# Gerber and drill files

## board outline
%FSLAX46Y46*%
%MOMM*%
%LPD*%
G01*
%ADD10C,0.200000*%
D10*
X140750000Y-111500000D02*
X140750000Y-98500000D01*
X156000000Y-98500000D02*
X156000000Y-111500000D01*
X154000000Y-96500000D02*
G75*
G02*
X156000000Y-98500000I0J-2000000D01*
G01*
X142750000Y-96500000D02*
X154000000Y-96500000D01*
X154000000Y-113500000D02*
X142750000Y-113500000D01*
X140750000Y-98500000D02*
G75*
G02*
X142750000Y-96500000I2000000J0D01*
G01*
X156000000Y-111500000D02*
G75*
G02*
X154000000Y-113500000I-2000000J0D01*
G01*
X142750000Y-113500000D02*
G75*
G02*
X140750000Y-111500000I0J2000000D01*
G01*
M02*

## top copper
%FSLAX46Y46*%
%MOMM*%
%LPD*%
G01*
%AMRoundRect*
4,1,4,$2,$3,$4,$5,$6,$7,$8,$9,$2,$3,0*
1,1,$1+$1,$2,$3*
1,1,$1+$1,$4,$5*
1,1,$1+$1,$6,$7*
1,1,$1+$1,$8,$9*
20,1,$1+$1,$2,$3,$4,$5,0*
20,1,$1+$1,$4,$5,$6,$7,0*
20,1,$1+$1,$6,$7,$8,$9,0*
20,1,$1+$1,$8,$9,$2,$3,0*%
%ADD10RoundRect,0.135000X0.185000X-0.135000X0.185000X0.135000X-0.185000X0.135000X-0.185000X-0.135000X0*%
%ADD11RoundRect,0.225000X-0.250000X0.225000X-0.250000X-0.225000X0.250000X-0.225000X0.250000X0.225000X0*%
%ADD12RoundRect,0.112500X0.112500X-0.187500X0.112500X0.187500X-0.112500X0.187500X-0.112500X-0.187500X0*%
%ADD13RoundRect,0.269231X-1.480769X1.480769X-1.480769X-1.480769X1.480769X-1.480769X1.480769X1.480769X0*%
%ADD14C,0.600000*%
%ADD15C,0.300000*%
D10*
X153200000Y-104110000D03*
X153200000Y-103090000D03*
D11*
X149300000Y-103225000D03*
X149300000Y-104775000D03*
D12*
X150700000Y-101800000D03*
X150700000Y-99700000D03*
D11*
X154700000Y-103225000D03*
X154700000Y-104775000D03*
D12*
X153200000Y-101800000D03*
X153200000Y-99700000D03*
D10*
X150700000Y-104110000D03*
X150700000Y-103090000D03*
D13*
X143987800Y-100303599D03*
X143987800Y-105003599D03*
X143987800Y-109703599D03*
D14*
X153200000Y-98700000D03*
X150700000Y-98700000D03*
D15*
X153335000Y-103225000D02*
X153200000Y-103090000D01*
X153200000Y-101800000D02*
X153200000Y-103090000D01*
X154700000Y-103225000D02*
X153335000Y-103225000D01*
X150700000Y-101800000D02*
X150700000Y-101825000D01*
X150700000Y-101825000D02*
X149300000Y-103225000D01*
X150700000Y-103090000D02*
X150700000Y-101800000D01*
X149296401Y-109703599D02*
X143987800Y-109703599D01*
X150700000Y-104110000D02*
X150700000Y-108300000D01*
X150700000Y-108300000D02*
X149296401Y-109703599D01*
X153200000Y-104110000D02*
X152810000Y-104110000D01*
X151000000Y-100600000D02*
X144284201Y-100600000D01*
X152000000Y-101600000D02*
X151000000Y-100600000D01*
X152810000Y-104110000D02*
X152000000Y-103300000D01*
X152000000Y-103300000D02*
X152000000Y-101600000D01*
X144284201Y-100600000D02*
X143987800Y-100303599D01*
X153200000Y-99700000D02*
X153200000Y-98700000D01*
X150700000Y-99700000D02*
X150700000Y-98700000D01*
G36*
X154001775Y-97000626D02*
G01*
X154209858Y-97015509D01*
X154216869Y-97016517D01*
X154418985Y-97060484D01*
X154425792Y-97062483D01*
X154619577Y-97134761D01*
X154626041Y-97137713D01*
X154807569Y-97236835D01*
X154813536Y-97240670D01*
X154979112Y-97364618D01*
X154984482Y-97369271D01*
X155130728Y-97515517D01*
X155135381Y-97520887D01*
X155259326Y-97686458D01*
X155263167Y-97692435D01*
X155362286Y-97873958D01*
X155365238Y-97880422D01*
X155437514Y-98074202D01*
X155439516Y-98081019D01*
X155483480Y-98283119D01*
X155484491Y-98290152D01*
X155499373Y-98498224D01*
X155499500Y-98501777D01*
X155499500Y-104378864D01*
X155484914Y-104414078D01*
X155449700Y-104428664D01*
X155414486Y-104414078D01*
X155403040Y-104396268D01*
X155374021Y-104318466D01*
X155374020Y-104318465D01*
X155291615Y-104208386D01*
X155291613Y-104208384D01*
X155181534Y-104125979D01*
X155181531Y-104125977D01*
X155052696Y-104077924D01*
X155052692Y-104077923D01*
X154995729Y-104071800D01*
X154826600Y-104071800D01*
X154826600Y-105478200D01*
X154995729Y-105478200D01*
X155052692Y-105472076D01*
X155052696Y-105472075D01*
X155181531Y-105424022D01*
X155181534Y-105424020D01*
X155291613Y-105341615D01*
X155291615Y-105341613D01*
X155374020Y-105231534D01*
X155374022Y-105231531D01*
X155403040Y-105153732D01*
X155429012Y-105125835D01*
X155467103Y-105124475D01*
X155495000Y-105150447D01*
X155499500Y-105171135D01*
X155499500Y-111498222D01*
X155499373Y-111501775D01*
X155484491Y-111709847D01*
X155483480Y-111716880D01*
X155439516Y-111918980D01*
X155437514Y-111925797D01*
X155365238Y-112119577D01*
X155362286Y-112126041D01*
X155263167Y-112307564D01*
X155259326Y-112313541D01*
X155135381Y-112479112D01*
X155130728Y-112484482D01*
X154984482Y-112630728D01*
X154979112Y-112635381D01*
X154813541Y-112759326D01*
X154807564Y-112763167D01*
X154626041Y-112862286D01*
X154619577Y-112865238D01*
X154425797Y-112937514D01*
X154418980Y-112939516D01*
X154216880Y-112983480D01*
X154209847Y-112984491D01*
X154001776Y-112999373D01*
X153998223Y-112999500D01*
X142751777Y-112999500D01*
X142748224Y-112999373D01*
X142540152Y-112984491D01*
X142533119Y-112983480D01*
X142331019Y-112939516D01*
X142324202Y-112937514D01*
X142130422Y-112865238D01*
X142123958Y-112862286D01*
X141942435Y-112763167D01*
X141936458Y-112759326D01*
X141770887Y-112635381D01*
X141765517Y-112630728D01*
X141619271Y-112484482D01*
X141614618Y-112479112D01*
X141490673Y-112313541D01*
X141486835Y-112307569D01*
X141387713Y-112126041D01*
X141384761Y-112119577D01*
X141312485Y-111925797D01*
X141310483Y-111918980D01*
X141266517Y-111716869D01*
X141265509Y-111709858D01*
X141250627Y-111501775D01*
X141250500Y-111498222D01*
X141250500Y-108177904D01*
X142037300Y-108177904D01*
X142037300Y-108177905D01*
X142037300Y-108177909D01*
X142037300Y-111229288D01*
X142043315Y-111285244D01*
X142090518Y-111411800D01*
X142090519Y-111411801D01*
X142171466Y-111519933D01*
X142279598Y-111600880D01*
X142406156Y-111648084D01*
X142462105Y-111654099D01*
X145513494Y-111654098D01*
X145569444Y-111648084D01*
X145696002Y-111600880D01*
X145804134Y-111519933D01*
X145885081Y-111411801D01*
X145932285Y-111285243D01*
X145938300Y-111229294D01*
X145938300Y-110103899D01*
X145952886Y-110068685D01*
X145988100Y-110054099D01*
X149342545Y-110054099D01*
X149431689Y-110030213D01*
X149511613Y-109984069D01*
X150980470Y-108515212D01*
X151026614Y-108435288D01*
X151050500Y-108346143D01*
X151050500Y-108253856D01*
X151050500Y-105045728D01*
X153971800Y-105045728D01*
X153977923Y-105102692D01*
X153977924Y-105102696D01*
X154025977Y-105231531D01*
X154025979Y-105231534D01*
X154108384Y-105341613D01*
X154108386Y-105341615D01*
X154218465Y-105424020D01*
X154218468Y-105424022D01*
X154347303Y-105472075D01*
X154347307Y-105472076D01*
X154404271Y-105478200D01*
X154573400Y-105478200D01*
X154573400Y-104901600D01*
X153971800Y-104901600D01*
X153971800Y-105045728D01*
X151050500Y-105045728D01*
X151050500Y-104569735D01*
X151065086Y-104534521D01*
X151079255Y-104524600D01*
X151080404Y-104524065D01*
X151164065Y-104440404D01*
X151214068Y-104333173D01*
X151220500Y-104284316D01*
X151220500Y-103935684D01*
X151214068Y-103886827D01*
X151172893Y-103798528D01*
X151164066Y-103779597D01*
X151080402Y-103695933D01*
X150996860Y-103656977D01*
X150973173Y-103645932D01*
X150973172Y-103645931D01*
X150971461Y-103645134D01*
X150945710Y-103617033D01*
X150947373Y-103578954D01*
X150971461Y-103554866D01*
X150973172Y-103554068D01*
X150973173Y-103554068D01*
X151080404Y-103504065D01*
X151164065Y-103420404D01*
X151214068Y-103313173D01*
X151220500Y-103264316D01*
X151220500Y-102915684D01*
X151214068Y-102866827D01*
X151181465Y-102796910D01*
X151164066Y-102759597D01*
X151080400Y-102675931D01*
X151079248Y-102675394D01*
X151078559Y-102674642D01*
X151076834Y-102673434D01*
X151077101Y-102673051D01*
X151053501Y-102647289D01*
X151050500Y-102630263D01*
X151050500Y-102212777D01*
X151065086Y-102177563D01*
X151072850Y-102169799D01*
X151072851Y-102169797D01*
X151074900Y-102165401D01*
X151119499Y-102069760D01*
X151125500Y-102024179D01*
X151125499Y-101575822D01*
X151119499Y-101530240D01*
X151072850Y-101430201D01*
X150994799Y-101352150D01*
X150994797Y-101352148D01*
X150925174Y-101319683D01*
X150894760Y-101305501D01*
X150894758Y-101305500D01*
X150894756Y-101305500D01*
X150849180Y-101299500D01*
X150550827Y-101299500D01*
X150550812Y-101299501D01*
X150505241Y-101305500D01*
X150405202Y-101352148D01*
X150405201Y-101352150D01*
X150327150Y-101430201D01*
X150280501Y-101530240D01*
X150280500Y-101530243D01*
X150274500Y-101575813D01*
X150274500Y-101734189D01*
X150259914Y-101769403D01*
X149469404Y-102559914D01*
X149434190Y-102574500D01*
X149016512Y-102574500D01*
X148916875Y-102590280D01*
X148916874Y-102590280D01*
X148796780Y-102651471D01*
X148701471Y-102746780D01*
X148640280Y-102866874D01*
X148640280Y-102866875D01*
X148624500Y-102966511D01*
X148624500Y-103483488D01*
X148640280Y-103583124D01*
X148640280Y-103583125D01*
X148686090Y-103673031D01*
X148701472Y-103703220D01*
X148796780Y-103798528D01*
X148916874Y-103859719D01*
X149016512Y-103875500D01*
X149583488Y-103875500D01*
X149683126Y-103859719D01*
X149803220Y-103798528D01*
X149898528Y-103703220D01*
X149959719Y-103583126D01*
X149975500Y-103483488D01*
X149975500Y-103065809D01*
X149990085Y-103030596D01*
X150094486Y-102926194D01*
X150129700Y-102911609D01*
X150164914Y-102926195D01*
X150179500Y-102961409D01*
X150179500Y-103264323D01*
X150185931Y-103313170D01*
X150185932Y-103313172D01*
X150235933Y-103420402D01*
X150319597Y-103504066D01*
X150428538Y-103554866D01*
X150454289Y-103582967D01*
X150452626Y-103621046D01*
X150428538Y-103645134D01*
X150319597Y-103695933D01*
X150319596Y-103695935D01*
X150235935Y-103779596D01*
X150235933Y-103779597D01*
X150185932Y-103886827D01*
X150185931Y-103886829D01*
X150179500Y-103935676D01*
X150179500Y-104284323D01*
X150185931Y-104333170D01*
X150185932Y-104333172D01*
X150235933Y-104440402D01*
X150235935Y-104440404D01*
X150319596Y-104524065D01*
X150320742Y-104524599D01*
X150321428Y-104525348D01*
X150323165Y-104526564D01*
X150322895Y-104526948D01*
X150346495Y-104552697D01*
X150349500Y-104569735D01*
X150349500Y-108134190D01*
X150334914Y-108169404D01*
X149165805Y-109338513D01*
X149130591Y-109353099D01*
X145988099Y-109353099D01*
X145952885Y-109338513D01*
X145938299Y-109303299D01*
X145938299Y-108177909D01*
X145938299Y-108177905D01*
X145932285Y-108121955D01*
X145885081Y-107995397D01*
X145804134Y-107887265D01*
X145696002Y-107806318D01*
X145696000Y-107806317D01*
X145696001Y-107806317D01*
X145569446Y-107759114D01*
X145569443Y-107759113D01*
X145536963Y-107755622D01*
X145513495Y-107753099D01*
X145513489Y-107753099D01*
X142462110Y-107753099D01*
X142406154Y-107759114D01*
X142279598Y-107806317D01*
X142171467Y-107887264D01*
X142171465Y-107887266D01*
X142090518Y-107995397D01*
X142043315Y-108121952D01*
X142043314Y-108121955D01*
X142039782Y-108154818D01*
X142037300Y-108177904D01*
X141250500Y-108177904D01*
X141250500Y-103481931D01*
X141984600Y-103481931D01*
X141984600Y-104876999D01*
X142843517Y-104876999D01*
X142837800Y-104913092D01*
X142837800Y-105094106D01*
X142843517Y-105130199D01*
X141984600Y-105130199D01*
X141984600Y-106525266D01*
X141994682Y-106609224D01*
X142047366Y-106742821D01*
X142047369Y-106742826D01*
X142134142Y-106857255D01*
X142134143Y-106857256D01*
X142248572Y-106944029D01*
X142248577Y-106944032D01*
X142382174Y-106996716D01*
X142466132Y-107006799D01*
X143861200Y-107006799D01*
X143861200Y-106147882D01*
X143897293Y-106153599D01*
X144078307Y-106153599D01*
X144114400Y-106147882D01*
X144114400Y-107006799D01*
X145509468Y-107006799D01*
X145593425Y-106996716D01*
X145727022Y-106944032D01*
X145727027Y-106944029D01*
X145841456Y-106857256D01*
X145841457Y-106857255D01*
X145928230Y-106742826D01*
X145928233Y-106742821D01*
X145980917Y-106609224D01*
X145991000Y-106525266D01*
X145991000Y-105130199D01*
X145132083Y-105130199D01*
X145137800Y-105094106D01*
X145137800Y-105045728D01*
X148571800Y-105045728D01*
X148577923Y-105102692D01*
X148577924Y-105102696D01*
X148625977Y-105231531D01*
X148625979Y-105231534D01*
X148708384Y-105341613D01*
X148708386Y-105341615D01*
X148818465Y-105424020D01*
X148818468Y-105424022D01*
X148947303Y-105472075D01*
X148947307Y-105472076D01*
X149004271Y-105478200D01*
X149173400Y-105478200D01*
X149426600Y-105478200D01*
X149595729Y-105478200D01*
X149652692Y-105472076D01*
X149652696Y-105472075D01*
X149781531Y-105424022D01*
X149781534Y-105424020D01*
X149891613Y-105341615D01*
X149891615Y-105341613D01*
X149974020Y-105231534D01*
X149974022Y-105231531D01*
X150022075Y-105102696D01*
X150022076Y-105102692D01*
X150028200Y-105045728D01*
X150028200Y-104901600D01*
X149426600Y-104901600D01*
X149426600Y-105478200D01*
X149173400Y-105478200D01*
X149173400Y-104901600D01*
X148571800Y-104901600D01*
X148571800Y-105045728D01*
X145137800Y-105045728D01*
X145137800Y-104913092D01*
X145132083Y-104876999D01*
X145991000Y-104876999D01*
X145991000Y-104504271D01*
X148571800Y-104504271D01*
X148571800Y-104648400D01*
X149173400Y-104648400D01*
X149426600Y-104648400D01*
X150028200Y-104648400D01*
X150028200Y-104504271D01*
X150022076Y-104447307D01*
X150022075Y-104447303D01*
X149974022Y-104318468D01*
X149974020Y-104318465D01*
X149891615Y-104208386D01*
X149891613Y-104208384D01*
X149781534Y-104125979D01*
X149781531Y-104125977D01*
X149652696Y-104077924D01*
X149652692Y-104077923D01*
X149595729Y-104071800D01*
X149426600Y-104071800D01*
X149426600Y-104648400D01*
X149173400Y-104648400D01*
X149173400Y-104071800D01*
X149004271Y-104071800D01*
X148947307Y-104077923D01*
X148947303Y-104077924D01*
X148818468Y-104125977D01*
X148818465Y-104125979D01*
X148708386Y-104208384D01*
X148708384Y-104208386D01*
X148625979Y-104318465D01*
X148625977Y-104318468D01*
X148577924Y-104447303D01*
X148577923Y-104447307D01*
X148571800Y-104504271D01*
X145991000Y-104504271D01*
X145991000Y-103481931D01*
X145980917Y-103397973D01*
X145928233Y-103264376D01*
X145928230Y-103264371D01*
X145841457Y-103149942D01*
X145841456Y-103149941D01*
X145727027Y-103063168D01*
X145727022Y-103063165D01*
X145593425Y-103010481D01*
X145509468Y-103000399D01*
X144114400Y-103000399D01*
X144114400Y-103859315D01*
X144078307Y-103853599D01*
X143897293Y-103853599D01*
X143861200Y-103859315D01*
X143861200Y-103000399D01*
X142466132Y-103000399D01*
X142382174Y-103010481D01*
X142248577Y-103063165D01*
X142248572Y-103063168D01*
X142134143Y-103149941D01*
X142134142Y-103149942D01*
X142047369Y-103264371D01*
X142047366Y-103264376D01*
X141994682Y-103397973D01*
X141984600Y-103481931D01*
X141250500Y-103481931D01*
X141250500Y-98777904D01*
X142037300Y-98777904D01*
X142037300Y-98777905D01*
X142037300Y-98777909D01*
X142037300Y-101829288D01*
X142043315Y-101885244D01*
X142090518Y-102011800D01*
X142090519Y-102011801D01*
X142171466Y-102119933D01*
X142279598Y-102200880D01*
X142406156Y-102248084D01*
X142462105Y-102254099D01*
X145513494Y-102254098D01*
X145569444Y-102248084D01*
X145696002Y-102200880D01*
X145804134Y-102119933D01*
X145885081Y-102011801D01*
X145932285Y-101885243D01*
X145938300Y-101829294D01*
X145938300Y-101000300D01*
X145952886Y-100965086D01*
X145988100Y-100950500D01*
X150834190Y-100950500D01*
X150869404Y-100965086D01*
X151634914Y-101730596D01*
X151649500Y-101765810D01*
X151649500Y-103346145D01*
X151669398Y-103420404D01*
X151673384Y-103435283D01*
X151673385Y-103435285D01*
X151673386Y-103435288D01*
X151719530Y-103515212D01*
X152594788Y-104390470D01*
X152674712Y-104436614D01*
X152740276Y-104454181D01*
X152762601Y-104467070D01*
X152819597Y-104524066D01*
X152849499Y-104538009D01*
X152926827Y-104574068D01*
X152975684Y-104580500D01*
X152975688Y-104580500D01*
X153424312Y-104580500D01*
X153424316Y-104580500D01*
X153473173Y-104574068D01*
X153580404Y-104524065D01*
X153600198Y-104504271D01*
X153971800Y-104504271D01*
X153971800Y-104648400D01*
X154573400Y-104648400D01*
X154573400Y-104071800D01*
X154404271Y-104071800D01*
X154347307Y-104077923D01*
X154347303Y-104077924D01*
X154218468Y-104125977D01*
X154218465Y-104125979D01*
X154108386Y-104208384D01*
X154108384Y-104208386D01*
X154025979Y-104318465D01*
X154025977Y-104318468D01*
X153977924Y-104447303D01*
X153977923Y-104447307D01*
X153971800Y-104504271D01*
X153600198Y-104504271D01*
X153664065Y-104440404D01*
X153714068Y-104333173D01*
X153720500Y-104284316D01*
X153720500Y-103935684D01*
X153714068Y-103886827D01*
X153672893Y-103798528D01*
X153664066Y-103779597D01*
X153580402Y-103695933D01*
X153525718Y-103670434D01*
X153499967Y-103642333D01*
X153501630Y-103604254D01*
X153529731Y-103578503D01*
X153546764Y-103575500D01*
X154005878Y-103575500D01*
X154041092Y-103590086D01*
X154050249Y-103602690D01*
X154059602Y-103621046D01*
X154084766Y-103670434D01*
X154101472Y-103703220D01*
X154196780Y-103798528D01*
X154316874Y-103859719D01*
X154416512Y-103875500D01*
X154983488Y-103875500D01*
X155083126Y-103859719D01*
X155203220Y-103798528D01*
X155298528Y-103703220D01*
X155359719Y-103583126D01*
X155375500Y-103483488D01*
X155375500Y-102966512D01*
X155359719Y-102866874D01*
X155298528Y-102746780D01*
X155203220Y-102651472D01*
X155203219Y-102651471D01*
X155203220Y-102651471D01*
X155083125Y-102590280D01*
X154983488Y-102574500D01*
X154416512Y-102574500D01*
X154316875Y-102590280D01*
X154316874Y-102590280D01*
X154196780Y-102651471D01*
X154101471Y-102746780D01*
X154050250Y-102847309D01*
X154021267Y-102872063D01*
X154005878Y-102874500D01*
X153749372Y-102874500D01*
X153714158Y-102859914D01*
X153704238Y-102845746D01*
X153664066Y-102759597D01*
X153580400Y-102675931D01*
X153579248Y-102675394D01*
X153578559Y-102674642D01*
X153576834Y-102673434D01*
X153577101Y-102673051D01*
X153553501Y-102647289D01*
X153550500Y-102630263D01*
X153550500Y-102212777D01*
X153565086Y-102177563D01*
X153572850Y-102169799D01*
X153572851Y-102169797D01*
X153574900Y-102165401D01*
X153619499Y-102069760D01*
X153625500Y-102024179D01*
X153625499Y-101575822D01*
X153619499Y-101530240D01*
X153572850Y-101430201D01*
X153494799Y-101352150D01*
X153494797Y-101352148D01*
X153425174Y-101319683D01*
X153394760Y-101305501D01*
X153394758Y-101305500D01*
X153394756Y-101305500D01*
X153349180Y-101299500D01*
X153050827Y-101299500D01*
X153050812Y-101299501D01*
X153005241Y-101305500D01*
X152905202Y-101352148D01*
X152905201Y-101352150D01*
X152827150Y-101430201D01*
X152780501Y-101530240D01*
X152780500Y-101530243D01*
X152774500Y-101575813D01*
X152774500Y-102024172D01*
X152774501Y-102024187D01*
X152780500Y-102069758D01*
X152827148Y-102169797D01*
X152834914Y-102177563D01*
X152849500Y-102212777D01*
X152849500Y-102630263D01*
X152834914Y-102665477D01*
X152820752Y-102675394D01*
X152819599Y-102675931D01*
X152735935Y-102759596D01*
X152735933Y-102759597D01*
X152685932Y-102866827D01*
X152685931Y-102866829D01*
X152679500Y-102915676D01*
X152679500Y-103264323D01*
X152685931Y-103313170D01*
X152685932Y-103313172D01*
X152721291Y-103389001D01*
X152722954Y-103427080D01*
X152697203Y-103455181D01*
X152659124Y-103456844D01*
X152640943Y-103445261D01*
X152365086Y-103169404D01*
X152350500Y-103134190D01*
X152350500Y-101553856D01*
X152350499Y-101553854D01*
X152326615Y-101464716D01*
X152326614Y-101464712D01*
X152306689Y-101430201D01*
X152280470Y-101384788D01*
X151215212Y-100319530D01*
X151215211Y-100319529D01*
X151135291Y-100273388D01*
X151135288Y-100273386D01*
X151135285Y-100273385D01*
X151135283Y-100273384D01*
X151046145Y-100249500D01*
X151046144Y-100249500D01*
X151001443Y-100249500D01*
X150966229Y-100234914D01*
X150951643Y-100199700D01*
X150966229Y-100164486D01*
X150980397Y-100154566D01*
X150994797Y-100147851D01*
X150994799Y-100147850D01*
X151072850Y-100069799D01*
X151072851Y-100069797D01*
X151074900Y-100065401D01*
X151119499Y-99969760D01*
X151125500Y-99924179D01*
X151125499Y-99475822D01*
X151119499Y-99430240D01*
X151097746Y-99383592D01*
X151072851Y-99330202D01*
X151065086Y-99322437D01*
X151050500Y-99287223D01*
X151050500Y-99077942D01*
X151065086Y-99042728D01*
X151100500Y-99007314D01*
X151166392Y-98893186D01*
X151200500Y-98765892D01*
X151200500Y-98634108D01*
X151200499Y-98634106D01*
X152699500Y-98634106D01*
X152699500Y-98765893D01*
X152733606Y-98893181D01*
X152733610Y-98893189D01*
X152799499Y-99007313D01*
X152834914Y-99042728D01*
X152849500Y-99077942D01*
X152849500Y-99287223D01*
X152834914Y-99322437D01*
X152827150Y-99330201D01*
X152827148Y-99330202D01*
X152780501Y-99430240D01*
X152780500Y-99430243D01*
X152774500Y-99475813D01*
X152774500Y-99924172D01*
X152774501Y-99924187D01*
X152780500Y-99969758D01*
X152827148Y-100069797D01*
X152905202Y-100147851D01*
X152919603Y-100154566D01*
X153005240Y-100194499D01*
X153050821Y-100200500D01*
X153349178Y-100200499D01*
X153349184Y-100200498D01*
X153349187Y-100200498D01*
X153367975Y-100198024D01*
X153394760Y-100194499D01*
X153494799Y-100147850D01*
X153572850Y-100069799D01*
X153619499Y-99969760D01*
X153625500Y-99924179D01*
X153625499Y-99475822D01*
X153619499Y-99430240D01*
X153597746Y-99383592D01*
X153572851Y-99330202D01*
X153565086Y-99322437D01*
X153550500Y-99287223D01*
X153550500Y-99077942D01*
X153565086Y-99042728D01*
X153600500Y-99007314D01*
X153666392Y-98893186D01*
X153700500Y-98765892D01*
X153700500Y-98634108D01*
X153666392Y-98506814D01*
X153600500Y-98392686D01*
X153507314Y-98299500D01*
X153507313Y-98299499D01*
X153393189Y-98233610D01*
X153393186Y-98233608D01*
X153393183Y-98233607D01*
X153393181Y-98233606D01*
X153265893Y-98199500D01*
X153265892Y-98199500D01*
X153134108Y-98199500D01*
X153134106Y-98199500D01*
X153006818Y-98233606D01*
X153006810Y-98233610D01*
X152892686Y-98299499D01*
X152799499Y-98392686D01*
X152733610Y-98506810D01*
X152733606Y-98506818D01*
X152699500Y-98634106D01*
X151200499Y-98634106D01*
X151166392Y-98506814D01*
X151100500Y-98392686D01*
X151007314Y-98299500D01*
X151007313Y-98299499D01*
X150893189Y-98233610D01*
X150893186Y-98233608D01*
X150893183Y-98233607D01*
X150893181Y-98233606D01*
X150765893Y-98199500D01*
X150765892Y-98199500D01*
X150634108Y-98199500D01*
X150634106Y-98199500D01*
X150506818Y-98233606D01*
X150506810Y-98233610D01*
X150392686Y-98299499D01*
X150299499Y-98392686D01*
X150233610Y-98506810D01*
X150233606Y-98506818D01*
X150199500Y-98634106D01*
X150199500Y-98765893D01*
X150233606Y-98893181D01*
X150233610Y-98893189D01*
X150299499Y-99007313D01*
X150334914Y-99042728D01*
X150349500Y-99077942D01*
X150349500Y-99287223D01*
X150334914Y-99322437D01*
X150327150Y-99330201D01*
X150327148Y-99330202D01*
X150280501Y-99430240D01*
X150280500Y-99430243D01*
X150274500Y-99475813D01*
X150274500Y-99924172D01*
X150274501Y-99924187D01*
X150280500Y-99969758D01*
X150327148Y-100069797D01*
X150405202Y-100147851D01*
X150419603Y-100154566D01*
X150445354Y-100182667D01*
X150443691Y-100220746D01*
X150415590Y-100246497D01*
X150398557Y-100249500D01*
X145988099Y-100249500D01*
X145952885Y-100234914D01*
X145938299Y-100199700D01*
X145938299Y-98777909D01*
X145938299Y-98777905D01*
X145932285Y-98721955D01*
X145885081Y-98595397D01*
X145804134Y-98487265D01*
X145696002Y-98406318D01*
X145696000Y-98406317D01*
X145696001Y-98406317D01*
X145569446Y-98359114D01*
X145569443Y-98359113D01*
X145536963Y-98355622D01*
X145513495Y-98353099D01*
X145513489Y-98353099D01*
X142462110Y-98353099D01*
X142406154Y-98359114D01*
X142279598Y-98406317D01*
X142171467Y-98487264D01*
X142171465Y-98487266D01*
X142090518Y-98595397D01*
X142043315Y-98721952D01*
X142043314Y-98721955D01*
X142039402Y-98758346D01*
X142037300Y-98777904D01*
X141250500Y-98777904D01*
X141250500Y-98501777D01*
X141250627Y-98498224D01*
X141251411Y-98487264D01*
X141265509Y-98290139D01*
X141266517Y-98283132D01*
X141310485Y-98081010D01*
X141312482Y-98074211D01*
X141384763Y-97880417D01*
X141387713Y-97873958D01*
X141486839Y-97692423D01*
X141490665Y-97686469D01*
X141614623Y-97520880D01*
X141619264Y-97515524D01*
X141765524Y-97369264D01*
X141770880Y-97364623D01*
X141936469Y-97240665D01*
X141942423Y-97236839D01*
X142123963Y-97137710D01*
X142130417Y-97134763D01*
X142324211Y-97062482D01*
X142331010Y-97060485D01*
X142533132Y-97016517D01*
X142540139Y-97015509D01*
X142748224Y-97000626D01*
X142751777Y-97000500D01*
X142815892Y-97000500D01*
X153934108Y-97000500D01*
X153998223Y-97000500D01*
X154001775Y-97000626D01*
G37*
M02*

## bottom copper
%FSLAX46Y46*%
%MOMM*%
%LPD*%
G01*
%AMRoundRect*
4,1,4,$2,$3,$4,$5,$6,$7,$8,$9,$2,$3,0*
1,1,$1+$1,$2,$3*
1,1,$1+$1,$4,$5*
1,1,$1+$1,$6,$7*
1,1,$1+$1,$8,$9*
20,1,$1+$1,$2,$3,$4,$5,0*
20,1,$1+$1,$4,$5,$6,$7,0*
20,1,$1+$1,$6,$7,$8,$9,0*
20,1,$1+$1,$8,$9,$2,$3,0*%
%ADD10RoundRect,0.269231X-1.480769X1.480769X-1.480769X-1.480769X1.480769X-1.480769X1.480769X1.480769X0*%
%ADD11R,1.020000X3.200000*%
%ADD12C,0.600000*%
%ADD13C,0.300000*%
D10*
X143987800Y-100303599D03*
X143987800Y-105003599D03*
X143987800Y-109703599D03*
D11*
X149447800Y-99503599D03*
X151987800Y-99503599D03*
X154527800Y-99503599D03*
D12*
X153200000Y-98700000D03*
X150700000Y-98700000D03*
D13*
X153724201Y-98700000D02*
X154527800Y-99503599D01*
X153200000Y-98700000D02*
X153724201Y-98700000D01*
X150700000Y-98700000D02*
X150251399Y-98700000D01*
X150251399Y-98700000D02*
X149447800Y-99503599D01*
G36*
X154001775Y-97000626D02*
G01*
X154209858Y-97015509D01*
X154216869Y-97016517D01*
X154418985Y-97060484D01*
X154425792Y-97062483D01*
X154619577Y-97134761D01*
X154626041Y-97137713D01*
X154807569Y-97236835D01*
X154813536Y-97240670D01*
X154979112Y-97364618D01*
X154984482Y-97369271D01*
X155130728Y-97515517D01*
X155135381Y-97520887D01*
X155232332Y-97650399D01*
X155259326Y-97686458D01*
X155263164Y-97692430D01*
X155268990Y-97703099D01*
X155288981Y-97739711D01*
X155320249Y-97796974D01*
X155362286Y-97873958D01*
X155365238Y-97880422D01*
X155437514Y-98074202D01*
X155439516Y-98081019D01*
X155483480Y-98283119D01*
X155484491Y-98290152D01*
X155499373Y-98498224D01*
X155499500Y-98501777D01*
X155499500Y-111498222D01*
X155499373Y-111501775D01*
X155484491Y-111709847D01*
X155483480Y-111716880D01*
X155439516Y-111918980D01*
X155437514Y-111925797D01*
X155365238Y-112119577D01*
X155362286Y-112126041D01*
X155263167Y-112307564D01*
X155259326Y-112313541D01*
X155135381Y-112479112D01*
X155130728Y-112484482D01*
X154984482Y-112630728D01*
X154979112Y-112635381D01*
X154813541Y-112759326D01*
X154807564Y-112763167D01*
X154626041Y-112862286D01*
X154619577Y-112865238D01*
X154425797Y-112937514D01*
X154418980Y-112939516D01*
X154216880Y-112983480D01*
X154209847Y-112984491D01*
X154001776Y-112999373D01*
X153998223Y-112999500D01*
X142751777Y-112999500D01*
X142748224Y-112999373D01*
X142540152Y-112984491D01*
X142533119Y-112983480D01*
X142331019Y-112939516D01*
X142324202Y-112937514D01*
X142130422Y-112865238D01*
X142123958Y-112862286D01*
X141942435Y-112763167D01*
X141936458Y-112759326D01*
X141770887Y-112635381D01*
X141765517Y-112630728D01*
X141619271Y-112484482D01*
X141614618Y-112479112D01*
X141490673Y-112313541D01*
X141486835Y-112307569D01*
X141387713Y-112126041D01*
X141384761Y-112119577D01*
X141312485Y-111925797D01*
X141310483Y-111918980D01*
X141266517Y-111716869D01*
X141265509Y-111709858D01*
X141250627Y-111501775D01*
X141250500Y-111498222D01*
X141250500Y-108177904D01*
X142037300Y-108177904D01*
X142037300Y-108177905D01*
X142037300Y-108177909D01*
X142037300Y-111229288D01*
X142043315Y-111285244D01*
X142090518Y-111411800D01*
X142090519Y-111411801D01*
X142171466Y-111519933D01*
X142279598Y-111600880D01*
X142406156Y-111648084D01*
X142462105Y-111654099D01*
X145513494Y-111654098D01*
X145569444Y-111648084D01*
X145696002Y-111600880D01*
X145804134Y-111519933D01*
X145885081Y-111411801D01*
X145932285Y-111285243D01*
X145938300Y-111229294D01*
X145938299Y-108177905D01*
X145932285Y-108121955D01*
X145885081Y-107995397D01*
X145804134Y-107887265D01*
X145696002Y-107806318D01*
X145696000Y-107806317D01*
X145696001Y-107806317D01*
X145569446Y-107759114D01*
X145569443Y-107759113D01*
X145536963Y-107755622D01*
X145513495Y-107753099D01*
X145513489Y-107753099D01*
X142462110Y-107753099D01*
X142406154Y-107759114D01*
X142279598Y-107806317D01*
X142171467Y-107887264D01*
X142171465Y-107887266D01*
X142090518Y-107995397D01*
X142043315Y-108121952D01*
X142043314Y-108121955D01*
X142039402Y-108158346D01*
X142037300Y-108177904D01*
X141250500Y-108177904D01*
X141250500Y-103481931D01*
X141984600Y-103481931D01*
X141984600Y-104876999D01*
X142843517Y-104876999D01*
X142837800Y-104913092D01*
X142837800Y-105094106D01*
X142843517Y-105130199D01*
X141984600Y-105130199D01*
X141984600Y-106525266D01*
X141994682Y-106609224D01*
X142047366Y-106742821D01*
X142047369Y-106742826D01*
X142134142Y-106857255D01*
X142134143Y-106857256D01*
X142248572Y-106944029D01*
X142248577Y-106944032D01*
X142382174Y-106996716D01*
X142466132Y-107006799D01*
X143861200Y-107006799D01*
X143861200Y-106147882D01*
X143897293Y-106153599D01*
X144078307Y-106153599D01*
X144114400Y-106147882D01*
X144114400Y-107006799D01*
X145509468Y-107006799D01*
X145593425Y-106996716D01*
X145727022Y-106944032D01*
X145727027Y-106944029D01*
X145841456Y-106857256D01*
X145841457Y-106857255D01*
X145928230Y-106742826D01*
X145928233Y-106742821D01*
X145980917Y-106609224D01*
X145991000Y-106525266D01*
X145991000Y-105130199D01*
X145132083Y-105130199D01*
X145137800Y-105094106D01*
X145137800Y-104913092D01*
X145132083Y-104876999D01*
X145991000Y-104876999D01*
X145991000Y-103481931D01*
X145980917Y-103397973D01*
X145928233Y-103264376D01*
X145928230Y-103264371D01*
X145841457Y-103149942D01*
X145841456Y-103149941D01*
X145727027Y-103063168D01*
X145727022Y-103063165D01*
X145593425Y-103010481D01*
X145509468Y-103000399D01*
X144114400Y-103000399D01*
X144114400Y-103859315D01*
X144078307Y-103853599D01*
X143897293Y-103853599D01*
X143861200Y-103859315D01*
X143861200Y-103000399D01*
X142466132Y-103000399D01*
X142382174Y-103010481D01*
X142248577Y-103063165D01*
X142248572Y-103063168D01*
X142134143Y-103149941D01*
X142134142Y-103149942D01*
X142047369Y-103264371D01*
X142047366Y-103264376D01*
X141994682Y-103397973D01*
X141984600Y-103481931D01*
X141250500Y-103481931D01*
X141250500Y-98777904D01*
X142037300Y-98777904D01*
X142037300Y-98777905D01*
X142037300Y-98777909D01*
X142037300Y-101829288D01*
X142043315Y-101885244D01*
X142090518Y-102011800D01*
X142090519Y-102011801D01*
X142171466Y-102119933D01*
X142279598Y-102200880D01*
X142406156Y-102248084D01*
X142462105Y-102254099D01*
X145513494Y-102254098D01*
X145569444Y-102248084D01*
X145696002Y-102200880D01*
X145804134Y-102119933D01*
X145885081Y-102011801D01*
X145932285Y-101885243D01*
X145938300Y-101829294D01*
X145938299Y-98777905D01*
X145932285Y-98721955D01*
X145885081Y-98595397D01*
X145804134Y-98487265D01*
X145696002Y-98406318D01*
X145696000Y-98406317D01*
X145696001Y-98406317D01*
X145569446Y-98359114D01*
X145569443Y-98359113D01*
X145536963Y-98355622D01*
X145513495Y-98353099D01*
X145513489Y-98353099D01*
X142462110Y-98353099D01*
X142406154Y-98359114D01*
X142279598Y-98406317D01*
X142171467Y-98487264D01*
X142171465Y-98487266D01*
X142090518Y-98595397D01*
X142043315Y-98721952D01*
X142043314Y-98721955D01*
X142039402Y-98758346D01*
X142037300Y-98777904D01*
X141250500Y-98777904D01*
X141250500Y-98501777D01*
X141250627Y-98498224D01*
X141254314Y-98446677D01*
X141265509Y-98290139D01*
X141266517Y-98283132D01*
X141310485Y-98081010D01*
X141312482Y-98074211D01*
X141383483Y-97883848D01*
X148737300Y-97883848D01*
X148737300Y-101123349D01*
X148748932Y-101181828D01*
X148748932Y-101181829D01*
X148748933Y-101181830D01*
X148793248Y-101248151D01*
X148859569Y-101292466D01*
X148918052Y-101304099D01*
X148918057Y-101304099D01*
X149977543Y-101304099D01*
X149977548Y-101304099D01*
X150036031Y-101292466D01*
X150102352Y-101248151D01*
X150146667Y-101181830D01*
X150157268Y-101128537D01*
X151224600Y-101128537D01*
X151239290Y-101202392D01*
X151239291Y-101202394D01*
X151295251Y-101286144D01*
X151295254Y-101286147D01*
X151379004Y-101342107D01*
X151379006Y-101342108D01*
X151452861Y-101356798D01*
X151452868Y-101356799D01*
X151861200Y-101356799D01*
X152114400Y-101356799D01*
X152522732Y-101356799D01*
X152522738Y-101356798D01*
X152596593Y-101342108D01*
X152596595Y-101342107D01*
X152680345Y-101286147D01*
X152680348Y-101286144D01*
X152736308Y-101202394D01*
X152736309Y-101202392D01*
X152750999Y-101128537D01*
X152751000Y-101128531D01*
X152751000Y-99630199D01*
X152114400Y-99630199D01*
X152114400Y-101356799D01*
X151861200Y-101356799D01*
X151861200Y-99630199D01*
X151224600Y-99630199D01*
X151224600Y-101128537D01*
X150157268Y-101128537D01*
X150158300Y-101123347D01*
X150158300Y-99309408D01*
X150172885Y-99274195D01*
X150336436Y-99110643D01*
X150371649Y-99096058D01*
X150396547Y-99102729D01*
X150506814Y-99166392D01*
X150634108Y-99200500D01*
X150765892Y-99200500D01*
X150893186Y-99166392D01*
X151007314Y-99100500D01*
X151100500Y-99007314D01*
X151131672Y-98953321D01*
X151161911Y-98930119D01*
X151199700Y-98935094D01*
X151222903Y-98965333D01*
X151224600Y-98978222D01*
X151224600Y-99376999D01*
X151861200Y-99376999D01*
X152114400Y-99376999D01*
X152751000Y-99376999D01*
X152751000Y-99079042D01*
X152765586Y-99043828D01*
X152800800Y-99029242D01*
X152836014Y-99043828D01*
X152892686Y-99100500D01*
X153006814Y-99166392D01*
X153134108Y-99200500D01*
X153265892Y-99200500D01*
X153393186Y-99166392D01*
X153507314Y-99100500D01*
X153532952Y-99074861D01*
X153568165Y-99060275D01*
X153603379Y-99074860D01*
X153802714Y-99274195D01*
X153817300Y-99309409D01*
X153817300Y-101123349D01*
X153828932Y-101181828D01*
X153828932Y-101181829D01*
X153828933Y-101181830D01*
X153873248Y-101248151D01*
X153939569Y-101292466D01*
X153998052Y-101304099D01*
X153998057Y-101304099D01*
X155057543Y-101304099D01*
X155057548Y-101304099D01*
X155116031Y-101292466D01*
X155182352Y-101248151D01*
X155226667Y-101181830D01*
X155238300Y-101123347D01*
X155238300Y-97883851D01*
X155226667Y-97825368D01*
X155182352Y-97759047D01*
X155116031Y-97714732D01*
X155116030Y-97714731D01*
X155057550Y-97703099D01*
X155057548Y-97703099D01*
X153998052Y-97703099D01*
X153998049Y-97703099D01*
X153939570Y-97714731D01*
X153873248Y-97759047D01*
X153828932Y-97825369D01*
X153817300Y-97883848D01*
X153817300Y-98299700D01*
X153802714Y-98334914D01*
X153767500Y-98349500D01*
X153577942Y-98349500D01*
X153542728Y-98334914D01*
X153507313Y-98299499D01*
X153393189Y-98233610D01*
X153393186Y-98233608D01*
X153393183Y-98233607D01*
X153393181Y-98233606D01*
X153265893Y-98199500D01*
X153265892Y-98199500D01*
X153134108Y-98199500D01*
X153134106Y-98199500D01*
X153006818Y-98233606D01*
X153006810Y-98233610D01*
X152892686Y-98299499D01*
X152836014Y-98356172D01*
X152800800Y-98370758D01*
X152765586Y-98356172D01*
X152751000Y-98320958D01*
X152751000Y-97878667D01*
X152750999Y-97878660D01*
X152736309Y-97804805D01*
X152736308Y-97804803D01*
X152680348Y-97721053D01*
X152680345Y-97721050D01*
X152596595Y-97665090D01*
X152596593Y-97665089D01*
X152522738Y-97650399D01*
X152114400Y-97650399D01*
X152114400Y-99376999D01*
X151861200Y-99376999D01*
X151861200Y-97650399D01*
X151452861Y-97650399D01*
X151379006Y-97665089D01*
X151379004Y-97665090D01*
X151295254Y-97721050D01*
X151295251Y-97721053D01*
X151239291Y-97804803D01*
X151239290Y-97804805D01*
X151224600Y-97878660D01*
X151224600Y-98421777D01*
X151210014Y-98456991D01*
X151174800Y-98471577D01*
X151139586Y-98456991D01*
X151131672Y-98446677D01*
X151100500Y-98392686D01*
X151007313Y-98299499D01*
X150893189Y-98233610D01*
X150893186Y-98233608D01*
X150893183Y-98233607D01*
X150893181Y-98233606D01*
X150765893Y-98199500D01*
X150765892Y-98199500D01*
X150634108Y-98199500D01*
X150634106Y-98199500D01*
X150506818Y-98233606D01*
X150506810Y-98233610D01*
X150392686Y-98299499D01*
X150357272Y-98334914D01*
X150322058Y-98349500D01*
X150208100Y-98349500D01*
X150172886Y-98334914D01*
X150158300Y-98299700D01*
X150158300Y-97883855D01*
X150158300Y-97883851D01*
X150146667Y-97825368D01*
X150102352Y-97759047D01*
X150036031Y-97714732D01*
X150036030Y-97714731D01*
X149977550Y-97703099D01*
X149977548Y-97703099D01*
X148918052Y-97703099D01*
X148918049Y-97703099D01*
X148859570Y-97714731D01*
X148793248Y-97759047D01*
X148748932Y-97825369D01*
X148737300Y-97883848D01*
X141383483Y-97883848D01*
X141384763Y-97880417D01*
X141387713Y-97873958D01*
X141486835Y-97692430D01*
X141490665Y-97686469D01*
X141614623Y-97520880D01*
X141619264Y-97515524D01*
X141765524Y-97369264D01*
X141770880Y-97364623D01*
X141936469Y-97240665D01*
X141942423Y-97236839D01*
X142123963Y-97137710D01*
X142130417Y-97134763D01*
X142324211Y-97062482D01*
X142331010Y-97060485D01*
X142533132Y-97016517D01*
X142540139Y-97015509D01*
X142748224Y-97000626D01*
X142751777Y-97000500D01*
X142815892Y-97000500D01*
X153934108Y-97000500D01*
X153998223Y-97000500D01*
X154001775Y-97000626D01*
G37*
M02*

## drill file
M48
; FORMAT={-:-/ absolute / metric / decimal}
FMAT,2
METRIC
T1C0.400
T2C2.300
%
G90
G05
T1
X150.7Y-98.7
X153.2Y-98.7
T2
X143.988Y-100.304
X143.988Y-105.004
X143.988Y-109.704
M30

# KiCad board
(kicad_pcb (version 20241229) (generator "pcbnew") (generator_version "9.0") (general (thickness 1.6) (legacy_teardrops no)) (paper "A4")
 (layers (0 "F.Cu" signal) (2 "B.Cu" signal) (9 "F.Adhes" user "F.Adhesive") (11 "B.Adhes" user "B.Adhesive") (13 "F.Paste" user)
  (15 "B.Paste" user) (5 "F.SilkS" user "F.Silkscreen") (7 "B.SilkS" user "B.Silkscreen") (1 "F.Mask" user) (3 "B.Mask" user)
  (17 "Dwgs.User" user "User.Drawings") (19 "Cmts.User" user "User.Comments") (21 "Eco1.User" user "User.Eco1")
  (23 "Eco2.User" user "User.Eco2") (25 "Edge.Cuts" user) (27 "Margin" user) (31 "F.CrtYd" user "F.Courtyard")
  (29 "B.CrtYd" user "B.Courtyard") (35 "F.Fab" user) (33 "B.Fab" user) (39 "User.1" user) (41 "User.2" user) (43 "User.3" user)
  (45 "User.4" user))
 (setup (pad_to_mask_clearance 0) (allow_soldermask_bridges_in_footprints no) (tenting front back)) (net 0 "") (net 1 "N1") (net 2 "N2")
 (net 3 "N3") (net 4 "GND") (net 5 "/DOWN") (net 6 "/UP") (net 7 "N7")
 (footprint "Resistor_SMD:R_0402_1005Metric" (layer "F.Cu") (at 153.2 103.6 90)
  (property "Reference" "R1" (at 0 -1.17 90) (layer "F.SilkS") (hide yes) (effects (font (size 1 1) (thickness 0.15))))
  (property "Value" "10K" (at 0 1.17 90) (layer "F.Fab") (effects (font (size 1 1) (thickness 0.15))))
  (pad "1" smd roundrect (at -0.51 0 90) (size 0.54 0.64) (layers "F.Cu" "F.Mask" "F.Paste") (roundrect_rratio 0.25) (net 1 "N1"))
  (pad "2" smd roundrect (at 0.51 0 90) (size 0.54 0.64) (layers "F.Cu" "F.Mask" "F.Paste") (roundrect_rratio 0.25) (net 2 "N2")))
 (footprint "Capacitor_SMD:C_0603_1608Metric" (layer "F.Cu") (at 149.3 104 -90)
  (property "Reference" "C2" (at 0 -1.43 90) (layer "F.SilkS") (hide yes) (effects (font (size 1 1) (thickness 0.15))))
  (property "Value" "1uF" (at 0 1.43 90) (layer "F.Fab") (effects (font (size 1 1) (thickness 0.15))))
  (pad "1" smd roundrect (at -0.775 0 270) (size 0.9 0.95) (layers "F.Cu" "F.Mask" "F.Paste") (roundrect_rratio 0.25) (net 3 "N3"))
  (pad "2" smd roundrect (at 0.775 0 270) (size 0.9 0.95) (layers "F.Cu" "F.Mask" "F.Paste") (roundrect_rratio 0.25) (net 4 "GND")))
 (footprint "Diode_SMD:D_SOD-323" (layer "F.Cu") (at 150.7 100.75 90)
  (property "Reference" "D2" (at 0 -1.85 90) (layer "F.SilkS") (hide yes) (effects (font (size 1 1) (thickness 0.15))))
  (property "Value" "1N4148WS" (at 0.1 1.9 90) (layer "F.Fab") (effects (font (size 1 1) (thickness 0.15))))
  (pad "1" smd roundrect (at -1.05 0 90) (size 0.6 0.45) (layers "F.Cu" "F.Mask" "F.Paste") (roundrect_rratio 0.25) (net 3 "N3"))
  (pad "2" smd roundrect (at 1.05 0 90) (size 0.6 0.45) (layers "F.Cu" "F.Mask" "F.Paste") (roundrect_rratio 0.25) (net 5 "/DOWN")))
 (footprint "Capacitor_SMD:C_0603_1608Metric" (layer "F.Cu") (at 154.7 104 -90)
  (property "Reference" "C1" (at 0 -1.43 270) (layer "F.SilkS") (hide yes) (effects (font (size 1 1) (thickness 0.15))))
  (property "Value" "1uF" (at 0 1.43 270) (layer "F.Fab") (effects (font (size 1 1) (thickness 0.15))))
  (pad "1" smd roundrect (at -0.775 0 270) (size 0.9 0.95) (layers "F.Cu" "F.Mask" "F.Paste") (roundrect_rratio 0.25) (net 2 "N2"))
  (pad "2" smd roundrect (at 0.775 0 270) (size 0.9 0.95) (layers "F.Cu" "F.Mask" "F.Paste") (roundrect_rratio 0.25) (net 4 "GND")))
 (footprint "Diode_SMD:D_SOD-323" (layer "F.Cu") (at 153.2 100.75 90)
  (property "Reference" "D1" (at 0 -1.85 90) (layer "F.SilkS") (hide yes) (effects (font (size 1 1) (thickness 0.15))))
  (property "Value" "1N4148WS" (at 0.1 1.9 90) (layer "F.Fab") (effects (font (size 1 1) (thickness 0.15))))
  (pad "1" smd roundrect (at -1.05 0 90) (size 0.6 0.45) (layers "F.Cu" "F.Mask" "F.Paste") (roundrect_rratio 0.25) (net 2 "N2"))
  (pad "2" smd roundrect (at 1.05 0 90) (size 0.6 0.45) (layers "F.Cu" "F.Mask" "F.Paste") (roundrect_rratio 0.25) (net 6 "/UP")))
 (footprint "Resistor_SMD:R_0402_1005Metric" (layer "F.Cu") (at 150.7 103.6 90)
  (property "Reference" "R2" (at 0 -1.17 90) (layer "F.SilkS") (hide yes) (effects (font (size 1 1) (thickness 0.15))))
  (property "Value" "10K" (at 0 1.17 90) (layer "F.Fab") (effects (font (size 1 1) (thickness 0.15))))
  (pad "1" smd roundrect (at -0.51 0 90) (size 0.54 0.64) (layers "F.Cu" "F.Mask" "F.Paste") (roundrect_rratio 0.25) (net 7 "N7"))
  (pad "2" smd roundrect (at 0.51 0 90) (size 0.54 0.64) (layers "F.Cu" "F.Mask" "F.Paste") (roundrect_rratio 0.25) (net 3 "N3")))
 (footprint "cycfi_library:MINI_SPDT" (layer "F.Cu") (at 143.9878 105.003599 -90)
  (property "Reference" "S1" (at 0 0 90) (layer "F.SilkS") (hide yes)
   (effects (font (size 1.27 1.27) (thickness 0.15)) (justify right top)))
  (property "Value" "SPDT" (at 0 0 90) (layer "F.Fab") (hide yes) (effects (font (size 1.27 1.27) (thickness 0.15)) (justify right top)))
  (pad "1" thru_hole roundrect (at -4.7 0 270) (size 3.5 3.5) (drill 2.3) (layers "*.Cu" "*.Mask") (remove_unused_layers no)
   (roundrect_rratio 0.07692307692) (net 1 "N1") (solder_mask_margin 0) (thermal_bridge_angle 0))
  (pad "2" thru_hole roundrect (at 0 0 270) (size 3.5 3.5) (drill 2.3) (layers "*.Cu" "*.Mask") (remove_unused_layers no)
   (roundrect_rratio 0.07692307692) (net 4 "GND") (solder_mask_margin 0) (thermal_bridge_angle 0))
  (pad "3" thru_hole roundrect (at 4.7 0 270) (size 3.5 3.5) (drill 2.3) (layers "*.Cu" "*.Mask") (remove_unused_layers no)
   (roundrect_rratio 0.07692307692) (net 7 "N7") (solder_mask_margin 0) (thermal_bridge_angle 0)))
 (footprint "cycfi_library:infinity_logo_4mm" (layer "F.Cu") (at 150 111 90)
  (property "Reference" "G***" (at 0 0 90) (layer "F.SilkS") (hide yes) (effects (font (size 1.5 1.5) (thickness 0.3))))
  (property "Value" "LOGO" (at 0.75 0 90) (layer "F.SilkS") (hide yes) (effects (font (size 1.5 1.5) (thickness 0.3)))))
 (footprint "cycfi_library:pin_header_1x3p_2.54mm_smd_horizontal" (layer "B.Cu") (at 151.9878 99.503599 -90)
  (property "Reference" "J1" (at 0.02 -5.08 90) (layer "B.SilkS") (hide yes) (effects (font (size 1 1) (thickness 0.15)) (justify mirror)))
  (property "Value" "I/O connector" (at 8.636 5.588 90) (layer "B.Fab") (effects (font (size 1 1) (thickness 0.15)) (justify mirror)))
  (pad "1" smd rect (at 0 2.54 270) (size 3.2 1.02) (layers "B.Cu" "B.Mask" "B.Paste") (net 5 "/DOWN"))
  (pad "2" smd rect (at 0 0 270) (size 3.2 1.02) (layers "B.Cu" "B.Mask" "B.Paste") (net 4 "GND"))
  (pad "3" smd rect (at 0 -2.54 270) (size 3.2 1.02) (layers "B.Cu" "B.Mask" "B.Paste") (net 6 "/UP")))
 (gr_line (start 140.75 111.5) (end 140.75 98.5) (stroke (width 0.2) (type default)) (layer "Edge.Cuts"))
 (gr_line (start 156 98.5) (end 156 111.5) (stroke (width 0.2) (type default)) (layer "Edge.Cuts"))
 (gr_arc (start 154 96.5) (mid 155.414214 97.085786) (end 156 98.5) (stroke (width 0.2) (type default)) (layer "Edge.Cuts"))
 (gr_line (start 142.75 96.5) (end 154 96.5) (stroke (width 0.2) (type default)) (layer "Edge.Cuts"))
 (gr_line (start 154 113.5) (end 142.75 113.5) (stroke (width 0.2) (type default)) (layer "Edge.Cuts"))
 (gr_arc (start 140.75 98.5) (mid 141.335786 97.085786) (end 142.75 96.5) (stroke (width 0.2) (type default)) (layer "Edge.Cuts"))
 (gr_arc (start 156 111.5) (mid 155.414214 112.914214) (end 154 113.5) (stroke (width 0.2) (type default)) (layer "Edge.Cuts"))
 (gr_arc (start 142.75 113.5) (mid 141.335786 112.914214) (end 140.75 111.5) (stroke (width 0.2) (type default)) (layer "Edge.Cuts"))
 (segment (start 153.335 103.225) (end 153.2 103.09) (width 0.3) (layer "F.Cu") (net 2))
 (segment (start 153.2 101.8) (end 153.2 103.09) (width 0.3) (layer "F.Cu") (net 2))
 (segment (start 154.7 103.225) (end 153.335 103.225) (width 0.3) (layer "F.Cu") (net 2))
 (segment (start 150.7 101.8) (end 150.7 101.825) (width 0.3) (layer "F.Cu") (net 3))
 (segment (start 150.7 101.825) (end 149.3 103.225) (width 0.3) (layer "F.Cu") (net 3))
 (segment (start 150.7 103.09) (end 150.7 101.8) (width 0.3) (layer "F.Cu") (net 3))
 (segment (start 149.296401 109.703599) (end 143.9878 109.703599) (width 0.3) (layer "F.Cu") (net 7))
 (segment (start 150.7 104.11) (end 150.7 108.3) (width 0.3) (layer "F.Cu") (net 7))
 (segment (start 150.7 108.3) (end 149.296401 109.703599) (width 0.3) (layer "F.Cu") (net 7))
 (segment (start 153.2 104.11) (end 152.81 104.11) (width 0.3) (layer "F.Cu") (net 1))
 (segment (start 151 100.6) (end 144.284201 100.6) (width 0.3) (layer "F.Cu") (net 1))
 (segment (start 152 101.6) (end 151 100.6) (width 0.3) (layer "F.Cu") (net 1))
 (segment (start 152.81 104.11) (end 152 103.3) (width 0.3) (layer "F.Cu") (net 1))
 (segment (start 152 103.3) (end 152 101.6) (width 0.3) (layer "F.Cu") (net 1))
 (segment (start 144.284201 100.6) (end 143.9878 100.303599) (width 0.3) (layer "F.Cu") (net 1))
 (segment (start 153.2 99.7) (end 153.2 98.7) (width 0.3) (layer "F.Cu") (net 6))
 (via (at 153.2 98.7) (size 0.6) (drill 0.4) (layers "F.Cu" "B.Cu") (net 6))
 (segment (start 153.724201 98.7) (end 154.5278 99.503599) (width 0.3) (layer "B.Cu") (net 6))
 (segment (start 153.2 98.7) (end 153.724201 98.7) (width 0.3) (layer "B.Cu") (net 6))
 (segment (start 150.7 99.7) (end 150.7 98.7) (width 0.3) (layer "F.Cu") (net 5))
 (via (at 150.7 98.7) (size 0.6) (drill 0.4) (layers "F.Cu" "B.Cu") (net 5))
 (segment (start 150.7 98.7) (end 150.251399 98.7) (width 0.3) (layer "B.Cu") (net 5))
 (segment (start 150.251399 98.7) (end 149.4478 99.503599) (width 0.3) (layer "B.Cu") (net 5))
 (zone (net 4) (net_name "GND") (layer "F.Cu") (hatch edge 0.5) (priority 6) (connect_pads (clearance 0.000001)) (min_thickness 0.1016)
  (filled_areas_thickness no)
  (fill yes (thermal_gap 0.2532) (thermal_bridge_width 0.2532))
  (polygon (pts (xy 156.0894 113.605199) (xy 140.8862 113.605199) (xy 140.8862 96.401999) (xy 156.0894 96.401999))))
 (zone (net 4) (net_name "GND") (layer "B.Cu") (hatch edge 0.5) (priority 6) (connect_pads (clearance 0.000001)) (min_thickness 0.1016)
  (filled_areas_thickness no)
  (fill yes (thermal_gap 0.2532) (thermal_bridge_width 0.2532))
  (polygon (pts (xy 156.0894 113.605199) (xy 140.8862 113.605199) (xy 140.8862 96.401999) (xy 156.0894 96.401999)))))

